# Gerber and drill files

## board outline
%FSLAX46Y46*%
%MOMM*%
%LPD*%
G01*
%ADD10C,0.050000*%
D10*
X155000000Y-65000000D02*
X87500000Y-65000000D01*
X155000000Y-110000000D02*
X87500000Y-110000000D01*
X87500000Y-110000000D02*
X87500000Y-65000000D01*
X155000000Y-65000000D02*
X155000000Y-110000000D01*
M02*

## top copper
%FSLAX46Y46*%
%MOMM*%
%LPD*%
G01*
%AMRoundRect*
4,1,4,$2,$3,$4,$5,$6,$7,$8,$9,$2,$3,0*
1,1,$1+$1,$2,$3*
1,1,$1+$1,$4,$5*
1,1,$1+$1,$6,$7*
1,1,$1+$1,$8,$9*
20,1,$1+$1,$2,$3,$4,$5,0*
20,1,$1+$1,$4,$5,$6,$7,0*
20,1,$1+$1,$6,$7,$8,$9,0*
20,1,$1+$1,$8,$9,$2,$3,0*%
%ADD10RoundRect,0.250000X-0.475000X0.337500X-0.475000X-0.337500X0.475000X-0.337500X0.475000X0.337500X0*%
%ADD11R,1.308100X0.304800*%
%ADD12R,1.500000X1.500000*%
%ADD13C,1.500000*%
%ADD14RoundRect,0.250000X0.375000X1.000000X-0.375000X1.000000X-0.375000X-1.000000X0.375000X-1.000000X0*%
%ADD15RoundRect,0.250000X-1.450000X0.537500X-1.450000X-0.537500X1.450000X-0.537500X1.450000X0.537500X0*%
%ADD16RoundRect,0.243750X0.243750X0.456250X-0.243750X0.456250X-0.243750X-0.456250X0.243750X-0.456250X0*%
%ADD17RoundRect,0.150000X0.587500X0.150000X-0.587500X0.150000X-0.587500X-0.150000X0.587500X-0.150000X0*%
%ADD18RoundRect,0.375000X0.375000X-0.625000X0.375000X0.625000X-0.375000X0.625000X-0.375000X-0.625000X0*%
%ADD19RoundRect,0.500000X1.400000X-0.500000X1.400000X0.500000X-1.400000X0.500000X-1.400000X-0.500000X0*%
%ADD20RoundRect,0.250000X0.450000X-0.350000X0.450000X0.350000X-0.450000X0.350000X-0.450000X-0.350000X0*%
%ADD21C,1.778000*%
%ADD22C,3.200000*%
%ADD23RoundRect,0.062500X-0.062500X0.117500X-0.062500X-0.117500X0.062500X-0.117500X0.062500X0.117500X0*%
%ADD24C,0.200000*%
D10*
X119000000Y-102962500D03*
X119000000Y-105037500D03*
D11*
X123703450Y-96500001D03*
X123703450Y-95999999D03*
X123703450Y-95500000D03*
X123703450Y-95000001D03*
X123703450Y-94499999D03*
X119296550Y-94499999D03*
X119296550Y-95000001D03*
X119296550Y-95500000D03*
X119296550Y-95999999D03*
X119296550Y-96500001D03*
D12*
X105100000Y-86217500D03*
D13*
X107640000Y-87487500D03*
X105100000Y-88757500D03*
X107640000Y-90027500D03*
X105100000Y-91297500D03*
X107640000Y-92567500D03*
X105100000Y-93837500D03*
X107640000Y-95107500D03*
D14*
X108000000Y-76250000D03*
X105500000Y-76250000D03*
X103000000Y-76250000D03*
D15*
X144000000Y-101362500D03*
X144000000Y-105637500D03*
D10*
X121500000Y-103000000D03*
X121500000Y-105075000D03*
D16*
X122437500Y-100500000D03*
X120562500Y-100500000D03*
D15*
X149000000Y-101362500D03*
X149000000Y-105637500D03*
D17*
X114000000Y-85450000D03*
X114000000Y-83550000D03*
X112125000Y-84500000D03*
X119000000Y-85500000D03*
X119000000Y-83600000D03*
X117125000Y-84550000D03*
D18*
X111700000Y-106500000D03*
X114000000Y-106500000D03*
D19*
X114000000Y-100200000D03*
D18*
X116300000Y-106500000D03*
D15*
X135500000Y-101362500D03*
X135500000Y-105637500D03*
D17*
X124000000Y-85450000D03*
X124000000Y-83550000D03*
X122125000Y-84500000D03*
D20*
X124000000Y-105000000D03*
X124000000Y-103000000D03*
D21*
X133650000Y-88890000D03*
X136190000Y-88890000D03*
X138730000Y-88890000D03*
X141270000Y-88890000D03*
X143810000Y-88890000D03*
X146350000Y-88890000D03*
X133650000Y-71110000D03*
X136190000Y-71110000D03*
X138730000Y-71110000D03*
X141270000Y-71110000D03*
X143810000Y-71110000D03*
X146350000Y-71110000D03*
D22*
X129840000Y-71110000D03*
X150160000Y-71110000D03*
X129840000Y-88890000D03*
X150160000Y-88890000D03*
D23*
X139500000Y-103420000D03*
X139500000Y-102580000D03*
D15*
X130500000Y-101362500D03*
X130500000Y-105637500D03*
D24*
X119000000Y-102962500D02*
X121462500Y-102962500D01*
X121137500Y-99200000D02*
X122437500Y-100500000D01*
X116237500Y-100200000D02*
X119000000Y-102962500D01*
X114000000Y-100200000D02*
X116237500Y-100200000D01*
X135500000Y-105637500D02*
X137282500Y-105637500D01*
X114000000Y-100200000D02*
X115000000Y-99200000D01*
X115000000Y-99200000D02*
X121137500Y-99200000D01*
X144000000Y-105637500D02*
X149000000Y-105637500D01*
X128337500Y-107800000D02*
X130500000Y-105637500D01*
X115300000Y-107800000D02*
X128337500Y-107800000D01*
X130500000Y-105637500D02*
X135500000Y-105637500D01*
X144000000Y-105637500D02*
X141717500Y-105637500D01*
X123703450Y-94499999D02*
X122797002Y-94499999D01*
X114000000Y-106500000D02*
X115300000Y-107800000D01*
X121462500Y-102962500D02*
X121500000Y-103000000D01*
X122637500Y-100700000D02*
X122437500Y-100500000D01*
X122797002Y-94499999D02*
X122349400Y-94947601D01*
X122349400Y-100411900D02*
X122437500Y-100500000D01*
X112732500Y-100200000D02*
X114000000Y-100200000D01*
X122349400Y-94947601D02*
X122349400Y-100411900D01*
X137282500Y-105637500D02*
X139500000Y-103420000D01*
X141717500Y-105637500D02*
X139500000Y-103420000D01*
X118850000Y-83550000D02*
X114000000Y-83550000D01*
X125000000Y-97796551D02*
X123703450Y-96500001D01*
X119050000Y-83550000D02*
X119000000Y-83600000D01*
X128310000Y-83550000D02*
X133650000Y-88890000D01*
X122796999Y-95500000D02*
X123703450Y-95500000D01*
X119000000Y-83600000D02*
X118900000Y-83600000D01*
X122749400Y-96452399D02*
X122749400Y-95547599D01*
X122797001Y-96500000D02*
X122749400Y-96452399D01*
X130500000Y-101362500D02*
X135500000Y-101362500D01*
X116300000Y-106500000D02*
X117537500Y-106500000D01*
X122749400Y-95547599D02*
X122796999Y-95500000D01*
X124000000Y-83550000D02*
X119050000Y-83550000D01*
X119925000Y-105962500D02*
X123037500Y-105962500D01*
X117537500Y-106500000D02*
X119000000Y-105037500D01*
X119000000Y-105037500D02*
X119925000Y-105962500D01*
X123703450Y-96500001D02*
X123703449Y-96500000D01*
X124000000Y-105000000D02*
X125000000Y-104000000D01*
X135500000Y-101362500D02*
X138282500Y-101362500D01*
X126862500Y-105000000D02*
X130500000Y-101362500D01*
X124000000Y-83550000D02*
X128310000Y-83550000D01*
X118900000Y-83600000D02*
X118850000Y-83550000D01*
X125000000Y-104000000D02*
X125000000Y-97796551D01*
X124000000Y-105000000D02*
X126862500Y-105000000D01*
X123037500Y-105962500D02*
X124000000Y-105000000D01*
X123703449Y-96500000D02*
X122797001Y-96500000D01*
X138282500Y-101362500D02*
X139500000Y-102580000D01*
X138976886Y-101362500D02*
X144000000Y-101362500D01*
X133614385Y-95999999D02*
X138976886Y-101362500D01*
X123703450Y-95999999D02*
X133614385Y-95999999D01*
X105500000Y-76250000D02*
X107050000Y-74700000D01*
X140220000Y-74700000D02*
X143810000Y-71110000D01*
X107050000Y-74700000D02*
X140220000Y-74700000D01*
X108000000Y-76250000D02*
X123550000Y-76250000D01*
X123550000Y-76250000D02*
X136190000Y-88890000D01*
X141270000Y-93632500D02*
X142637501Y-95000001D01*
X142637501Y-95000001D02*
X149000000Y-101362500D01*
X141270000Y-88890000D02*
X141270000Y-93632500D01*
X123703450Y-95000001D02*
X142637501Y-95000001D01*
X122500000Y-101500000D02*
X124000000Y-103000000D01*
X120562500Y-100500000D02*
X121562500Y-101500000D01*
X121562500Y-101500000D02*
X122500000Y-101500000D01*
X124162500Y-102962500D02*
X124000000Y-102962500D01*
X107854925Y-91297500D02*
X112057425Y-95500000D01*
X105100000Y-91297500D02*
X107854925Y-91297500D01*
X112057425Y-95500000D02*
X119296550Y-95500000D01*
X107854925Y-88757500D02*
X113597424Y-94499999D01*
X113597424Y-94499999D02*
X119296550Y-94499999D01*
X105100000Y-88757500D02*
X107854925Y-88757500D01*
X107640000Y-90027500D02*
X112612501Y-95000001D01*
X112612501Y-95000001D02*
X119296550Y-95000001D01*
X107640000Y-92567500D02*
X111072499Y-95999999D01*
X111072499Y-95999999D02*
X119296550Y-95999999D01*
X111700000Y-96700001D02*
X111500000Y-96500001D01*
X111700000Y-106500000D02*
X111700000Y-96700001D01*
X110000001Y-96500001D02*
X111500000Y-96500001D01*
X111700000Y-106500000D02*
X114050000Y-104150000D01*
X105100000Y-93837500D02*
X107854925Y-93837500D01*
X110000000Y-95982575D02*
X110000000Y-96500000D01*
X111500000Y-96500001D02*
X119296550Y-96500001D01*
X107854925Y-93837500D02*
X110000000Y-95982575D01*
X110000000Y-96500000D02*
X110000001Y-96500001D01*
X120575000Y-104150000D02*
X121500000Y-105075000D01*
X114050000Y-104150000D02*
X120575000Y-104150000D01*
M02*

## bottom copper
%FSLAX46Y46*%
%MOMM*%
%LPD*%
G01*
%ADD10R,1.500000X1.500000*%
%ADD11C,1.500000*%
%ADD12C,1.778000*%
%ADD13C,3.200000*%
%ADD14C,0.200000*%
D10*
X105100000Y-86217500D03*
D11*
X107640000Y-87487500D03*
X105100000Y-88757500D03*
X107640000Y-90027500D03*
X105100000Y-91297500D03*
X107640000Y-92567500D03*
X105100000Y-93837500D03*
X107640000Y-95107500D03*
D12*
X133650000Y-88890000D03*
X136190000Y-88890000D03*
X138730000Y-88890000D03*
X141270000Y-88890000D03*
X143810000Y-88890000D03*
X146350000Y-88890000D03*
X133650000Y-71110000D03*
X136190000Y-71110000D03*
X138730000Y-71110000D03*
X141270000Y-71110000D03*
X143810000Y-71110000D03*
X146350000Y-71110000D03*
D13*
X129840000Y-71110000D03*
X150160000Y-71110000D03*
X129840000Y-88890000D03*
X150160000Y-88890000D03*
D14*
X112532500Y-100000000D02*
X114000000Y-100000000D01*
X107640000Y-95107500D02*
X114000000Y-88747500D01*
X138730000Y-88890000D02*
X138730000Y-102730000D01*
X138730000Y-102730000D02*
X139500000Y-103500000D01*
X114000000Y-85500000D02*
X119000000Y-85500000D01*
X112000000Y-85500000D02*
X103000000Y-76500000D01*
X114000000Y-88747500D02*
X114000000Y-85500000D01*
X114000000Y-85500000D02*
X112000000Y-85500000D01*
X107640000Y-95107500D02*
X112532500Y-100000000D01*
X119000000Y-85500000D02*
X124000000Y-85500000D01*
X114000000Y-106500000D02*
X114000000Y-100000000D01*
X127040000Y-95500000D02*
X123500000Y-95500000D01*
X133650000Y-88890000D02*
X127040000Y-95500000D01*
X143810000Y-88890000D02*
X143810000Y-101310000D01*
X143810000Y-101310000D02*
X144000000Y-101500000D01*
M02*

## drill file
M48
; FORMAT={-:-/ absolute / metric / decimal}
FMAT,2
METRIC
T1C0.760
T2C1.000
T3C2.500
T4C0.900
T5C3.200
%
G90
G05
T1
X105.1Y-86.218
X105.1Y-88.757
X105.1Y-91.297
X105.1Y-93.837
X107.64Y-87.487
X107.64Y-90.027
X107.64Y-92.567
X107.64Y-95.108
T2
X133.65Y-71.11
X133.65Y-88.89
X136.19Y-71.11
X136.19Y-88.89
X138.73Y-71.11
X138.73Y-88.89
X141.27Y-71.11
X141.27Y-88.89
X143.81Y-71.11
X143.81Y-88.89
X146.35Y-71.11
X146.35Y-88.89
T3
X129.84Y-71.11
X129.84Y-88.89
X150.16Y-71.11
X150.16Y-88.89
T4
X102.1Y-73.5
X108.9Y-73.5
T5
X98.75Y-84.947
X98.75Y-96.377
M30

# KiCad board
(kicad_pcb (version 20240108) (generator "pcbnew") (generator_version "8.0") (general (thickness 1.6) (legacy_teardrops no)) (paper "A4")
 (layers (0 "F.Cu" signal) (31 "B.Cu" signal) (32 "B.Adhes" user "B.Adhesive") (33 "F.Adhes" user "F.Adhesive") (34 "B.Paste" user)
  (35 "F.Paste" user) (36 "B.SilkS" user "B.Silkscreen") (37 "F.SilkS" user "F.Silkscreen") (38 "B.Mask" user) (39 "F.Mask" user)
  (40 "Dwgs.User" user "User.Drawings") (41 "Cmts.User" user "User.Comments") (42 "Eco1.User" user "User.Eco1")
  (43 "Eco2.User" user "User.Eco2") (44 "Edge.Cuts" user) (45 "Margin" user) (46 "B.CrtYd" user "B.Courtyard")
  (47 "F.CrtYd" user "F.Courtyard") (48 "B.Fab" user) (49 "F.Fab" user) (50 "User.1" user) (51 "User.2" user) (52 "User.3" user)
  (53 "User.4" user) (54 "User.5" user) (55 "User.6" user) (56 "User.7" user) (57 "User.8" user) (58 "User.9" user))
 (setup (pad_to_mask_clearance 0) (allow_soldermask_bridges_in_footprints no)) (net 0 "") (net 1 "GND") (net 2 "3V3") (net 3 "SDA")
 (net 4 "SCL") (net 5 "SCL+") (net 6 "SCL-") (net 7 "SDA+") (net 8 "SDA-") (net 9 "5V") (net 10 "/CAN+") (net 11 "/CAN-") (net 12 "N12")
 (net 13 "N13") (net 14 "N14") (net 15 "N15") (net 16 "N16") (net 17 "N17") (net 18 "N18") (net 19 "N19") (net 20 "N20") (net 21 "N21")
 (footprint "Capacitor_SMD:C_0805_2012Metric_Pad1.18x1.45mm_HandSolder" (layer "F.Cu") (at 119 104 -90)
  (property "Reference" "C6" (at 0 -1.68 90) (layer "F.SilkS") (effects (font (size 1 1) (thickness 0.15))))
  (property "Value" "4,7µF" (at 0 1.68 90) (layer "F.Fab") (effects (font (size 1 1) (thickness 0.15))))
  (pad "1" smd roundrect (at -1.0375 0 270) (size 1.175 1.45) (layers "F.Cu" "F.Paste" "F.Mask") (roundrect_rratio 0.212766) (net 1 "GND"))
  (pad "2" smd roundrect (at 1.0375 0 270) (size 1.175 1.45) (layers "F.Cu" "F.Paste" "F.Mask") (roundrect_rratio 0.212766) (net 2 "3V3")))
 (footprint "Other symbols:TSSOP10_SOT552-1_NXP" (layer "F.Cu") (at 121.5 95.5 180)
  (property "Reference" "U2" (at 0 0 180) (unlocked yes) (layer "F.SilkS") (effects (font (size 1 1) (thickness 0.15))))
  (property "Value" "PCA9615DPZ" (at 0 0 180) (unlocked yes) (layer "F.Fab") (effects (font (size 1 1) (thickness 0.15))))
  (pad "1" smd rect (at -2.20345 -1.000001 180) (size 1.3081 0.3048) (layers "F.Cu" "F.Paste" "F.Mask") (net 2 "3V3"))
  (pad "2" smd rect (at -2.20345 -0.499999 180) (size 1.3081 0.3048) (layers "F.Cu" "F.Paste" "F.Mask") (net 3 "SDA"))
  (pad "3" smd rect (at -2.20345 0 180) (size 1.3081 0.3048) (layers "F.Cu" "F.Paste" "F.Mask") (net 2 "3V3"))
  (pad "4" smd rect (at -2.20345 0.499999 180) (size 1.3081 0.3048) (layers "F.Cu" "F.Paste" "F.Mask") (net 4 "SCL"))
  (pad "5" smd rect (at -2.20345 1.000001 180) (size 1.3081 0.3048) (layers "F.Cu" "F.Paste" "F.Mask") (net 1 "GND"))
  (pad "6" smd rect (at 2.20345 1.000001 180) (size 1.3081 0.3048) (layers "F.Cu" "F.Paste" "F.Mask") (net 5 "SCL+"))
  (pad "7" smd rect (at 2.20345 0.499999 180) (size 1.3081 0.3048) (layers "F.Cu" "F.Paste" "F.Mask") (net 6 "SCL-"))
  (pad "8" smd rect (at 2.20345 0 180) (size 1.3081 0.3048) (layers "F.Cu" "F.Paste" "F.Mask") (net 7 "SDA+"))
  (pad "9" smd rect (at 2.20345 -0.499999 180) (size 1.3081 0.3048) (layers "F.Cu" "F.Paste" "F.Mask") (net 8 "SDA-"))
  (pad "10" smd rect (at 2.20345 -1.000001 180) (size 1.3081 0.3048) (layers "F.Cu" "F.Paste" "F.Mask") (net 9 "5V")))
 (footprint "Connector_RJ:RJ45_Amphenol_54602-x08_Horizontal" (layer "F.Cu") (at 105.1 86.2175 -90)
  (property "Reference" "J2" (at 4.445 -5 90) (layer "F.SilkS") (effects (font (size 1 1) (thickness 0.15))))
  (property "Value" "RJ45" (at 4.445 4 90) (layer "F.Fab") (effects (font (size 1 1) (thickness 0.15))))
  (pad "" np_thru_hole circle (at -1.27 6.35 270) (size 3.2 3.2) (drill 3.2) (layers "*.Cu" "*.Mask"))
  (pad "" np_thru_hole circle (at 10.16 6.35 270) (size 3.2 3.2) (drill 3.2) (layers "*.Cu" "*.Mask"))
  (pad "1" thru_hole rect (at 0 0 270) (size 1.5 1.5) (drill 0.76) (layers "*.Cu" "*.Mask") (remove_unused_layers no) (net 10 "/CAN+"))
  (pad "2" thru_hole circle (at 1.27 -2.54 270) (size 1.5 1.5) (drill 0.76) (layers "*.Cu" "*.Mask") (remove_unused_layers no)
   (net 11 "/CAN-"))
  (pad "3" thru_hole circle (at 2.54 0 270) (size 1.5 1.5) (drill 0.76) (layers "*.Cu" "*.Mask") (remove_unused_layers no) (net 5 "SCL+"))
  (pad "4" thru_hole circle (at 3.81 -2.54 270) (size 1.5 1.5) (drill 0.76) (layers "*.Cu" "*.Mask") (remove_unused_layers no)
   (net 6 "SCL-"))
  (pad "5" thru_hole circle (at 5.08 0 270) (size 1.5 1.5) (drill 0.76) (layers "*.Cu" "*.Mask") (remove_unused_layers no) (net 7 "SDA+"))
  (pad "6" thru_hole circle (at 6.35 -2.54 270) (size 1.5 1.5) (drill 0.76) (layers "*.Cu" "*.Mask") (remove_unused_layers no)
   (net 8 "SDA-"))
  (pad "7" thru_hole circle (at 7.62 0 270) (size 1.5 1.5) (drill 0.76) (layers "*.Cu" "*.Mask") (remove_unused_layers no) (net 9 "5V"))
  (pad "8" thru_hole circle (at 8.89 -2.54 270) (size 1.5 1.5) (drill 0.76) (layers "*.Cu" "*.Mask") (remove_unused_layers no) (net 1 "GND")))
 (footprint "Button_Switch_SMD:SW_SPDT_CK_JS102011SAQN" (layer "F.Cu") (at 105.5 73.5 180)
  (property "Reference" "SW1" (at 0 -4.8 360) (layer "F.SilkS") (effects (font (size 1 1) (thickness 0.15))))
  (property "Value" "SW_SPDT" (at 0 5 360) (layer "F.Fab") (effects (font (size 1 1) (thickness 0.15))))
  (pad "" np_thru_hole circle (at -3.4 0 180) (size 0.9 0.9) (drill 0.9) (layers "*.Cu" "*.Mask"))
  (pad "" np_thru_hole circle (at 3.4 0 180) (size 0.9 0.9) (drill 0.9) (layers "*.Cu" "*.Mask"))
  (pad "1" smd roundrect (at -2.5 -2.75 180) (size 1.25 2.5) (layers "F.Cu" "F.Paste" "F.Mask") (roundrect_rratio 0.2) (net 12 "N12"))
  (pad "2" smd roundrect (at 0 -2.75 180) (size 1.25 2.5) (layers "F.Cu" "F.Paste" "F.Mask") (roundrect_rratio 0.2) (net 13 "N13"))
  (pad "3" smd roundrect (at 2.5 -2.75 180) (size 1.25 2.5) (layers "F.Cu" "F.Paste" "F.Mask") (roundrect_rratio 0.2) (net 1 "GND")))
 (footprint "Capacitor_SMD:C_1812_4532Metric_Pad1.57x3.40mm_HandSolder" (layer "F.Cu") (at 144 103.5 -90)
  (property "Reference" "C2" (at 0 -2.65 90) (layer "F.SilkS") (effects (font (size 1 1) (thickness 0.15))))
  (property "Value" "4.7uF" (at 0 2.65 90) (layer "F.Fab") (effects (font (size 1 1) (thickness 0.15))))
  (pad "1" smd roundrect (at -2.1375 0 270) (size 1.575 3.4) (layers "F.Cu" "F.Paste" "F.Mask") (roundrect_rratio 0.15873) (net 3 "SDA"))
  (pad "2" smd roundrect (at 2.1375 0 270) (size 1.575 3.4) (layers "F.Cu" "F.Paste" "F.Mask") (roundrect_rratio 0.15873) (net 1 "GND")))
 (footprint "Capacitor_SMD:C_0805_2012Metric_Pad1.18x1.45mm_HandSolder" (layer "F.Cu") (at 121.5 104.0375 -90)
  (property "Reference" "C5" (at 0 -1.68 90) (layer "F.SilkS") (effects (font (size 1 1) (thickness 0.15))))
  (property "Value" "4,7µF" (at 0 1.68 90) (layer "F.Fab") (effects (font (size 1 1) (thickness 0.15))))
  (pad "1" smd roundrect (at -1.0375 0 270) (size 1.175 1.45) (layers "F.Cu" "F.Paste" "F.Mask") (roundrect_rratio 0.212766) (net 1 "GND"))
  (pad "2" smd roundrect (at 1.0375 0 270) (size 1.175 1.45) (layers "F.Cu" "F.Paste" "F.Mask") (roundrect_rratio 0.212766) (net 9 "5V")))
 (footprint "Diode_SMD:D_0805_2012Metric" (layer "F.Cu") (at 121.5 100.5 180)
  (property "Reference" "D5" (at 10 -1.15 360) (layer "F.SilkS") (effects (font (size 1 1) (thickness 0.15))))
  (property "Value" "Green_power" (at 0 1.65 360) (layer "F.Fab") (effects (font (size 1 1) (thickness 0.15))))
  (pad "1" smd roundrect (at -0.9375 0 180) (size 0.975 1.4) (layers "F.Cu" "F.Paste" "F.Mask") (roundrect_rratio 0.25) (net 1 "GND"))
  (pad "2" smd roundrect (at 0.9375 0 180) (size 0.975 1.4) (layers "F.Cu" "F.Paste" "F.Mask") (roundrect_rratio 0.25) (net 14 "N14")))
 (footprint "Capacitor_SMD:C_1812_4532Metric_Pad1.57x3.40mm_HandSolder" (layer "F.Cu") (at 149 103.5 -90)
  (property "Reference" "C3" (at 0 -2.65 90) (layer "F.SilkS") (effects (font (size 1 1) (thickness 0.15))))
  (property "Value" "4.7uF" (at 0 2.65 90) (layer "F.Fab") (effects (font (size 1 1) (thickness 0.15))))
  (pad "1" smd roundrect (at -2.1375 0 270) (size 1.575 3.4) (layers "F.Cu" "F.Paste" "F.Mask") (roundrect_rratio 0.15873) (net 4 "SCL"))
  (pad "2" smd roundrect (at 2.1375 0 270) (size 1.575 3.4) (layers "F.Cu" "F.Paste" "F.Mask") (roundrect_rratio 0.15873) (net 1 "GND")))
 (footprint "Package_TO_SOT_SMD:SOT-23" (layer "F.Cu") (at 113.0625 84.5 180)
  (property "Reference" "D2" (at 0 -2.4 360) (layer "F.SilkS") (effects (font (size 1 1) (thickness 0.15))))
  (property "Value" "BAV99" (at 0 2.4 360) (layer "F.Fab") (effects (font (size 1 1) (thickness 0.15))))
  (pad "1" smd roundrect (at -0.9375 -0.95 180) (size 1.475 0.6) (layers "F.Cu" "F.Paste" "F.Mask") (roundrect_rratio 0.25) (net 1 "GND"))
  (pad "2" smd roundrect (at -0.9375 0.95 180) (size 1.475 0.6) (layers "F.Cu" "F.Paste" "F.Mask") (roundrect_rratio 0.25) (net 2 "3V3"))
  (pad "3" smd roundrect (at 0.9375 0 180) (size 1.475 0.6) (layers "F.Cu" "F.Paste" "F.Mask") (roundrect_rratio 0.25) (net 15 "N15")))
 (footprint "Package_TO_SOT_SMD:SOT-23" (layer "F.Cu") (at 118.0625 84.55 180)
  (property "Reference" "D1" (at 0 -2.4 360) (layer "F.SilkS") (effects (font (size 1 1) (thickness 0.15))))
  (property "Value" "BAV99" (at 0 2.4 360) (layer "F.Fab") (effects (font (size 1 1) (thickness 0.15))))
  (pad "1" smd roundrect (at -0.9375 -0.95 180) (size 1.475 0.6) (layers "F.Cu" "F.Paste" "F.Mask") (roundrect_rratio 0.25) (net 1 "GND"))
  (pad "2" smd roundrect (at -0.9375 0.95 180) (size 1.475 0.6) (layers "F.Cu" "F.Paste" "F.Mask") (roundrect_rratio 0.25) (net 2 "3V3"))
  (pad "3" smd roundrect (at 0.9375 0 180) (size 1.475 0.6) (layers "F.Cu" "F.Paste" "F.Mask") (roundrect_rratio 0.25) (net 4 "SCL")))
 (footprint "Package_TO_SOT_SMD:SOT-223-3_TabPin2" (layer "F.Cu") (at 114 103.35 90)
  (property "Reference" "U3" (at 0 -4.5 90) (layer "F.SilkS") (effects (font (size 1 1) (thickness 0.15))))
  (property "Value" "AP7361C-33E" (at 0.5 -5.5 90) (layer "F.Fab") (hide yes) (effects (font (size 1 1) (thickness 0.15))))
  (pad "1" smd roundrect (at -3.15 -2.3 90) (size 2 1.5) (layers "F.Cu" "F.Paste" "F.Mask") (roundrect_rratio 0.25) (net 9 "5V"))
  (pad "2" smd roundrect (at -3.15 0 90) (size 2 1.5) (layers "F.Cu" "F.Paste" "F.Mask") (roundrect_rratio 0.25) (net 1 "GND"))
  (pad "2" smd roundrect (at 3.15 0 90) (size 2 3.8) (layers "F.Cu" "F.Paste" "F.Mask") (roundrect_rratio 0.25) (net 1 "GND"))
  (pad "3" smd roundrect (at -3.15 2.3 90) (size 2 1.5) (layers "F.Cu" "F.Paste" "F.Mask") (roundrect_rratio 0.25) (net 2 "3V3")))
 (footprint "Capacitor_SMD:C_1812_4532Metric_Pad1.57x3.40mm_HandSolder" (layer "F.Cu") (at 135.5 103.5 -90)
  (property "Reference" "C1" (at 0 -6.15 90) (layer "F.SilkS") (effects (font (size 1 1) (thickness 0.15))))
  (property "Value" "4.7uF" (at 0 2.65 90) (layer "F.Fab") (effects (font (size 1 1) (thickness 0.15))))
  (pad "1" smd roundrect (at -2.1375 0 270) (size 1.575 3.4) (layers "F.Cu" "F.Paste" "F.Mask") (roundrect_rratio 0.15873) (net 2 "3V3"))
  (pad "2" smd roundrect (at 2.1375 0 270) (size 1.575 3.4) (layers "F.Cu" "F.Paste" "F.Mask") (roundrect_rratio 0.15873) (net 1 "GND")))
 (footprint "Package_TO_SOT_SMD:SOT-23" (layer "F.Cu") (at 123.0625 84.5 180)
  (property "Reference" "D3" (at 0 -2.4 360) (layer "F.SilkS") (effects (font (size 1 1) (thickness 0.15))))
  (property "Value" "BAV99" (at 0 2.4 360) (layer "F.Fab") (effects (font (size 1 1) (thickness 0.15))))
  (pad "1" smd roundrect (at -0.9375 -0.95 180) (size 1.475 0.6) (layers "F.Cu" "F.Paste" "F.Mask") (roundrect_rratio 0.25) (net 1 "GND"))
  (pad "2" smd roundrect (at -0.9375 0.95 180) (size 1.475 0.6) (layers "F.Cu" "F.Paste" "F.Mask") (roundrect_rratio 0.25) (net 2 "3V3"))
  (pad "3" smd roundrect (at 0.9375 0 180) (size 1.475 0.6) (layers "F.Cu" "F.Paste" "F.Mask") (roundrect_rratio 0.25) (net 3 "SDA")))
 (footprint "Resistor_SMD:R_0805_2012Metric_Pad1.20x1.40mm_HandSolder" (layer "F.Cu") (at 124 104 90)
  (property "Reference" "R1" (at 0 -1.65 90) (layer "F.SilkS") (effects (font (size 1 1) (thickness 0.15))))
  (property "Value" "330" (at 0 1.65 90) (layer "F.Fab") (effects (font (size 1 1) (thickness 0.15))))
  (pad "1" smd roundrect (at -1 0 90) (size 1.2 1.4) (layers "F.Cu" "F.Paste" "F.Mask") (roundrect_rratio 0.208333) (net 2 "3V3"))
  (pad "2" smd roundrect (at 1 0 90) (size 1.2 1.4) (layers "F.Cu" "F.Paste" "F.Mask") (roundrect_rratio 0.208333) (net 14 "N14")))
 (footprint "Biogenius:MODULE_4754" (layer "F.Cu") (at 140 80)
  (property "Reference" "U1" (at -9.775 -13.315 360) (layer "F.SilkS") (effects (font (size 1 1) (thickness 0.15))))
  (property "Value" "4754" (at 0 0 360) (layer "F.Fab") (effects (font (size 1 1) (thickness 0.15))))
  (pad "JP1_1" thru_hole circle (at -6.35 8.89) (size 1.778 1.778) (drill 1) (layers "*.Cu" "*.Mask") (remove_unused_layers no)
   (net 2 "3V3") (solder_mask_margin 0.102))
  (pad "JP1_2" thru_hole circle (at -3.81 8.89) (size 1.778 1.778) (drill 1) (layers "*.Cu" "*.Mask") (remove_unused_layers no)
   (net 12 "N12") (solder_mask_margin 0.102))
  (pad "JP1_3" thru_hole circle (at -1.27 8.89) (size 1.778 1.778) (drill 1) (layers "*.Cu" "*.Mask") (remove_unused_layers no)
   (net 1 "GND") (solder_mask_margin 0.102))
  (pad "JP1_4" thru_hole circle (at 1.27 8.89) (size 1.778 1.778) (drill 1) (layers "*.Cu" "*.Mask") (remove_unused_layers no) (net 4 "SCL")
   (solder_mask_margin 0.102))
  (pad "JP1_5" thru_hole circle (at 3.81 8.89) (size 1.778 1.778) (drill 1) (layers "*.Cu" "*.Mask") (remove_unused_layers no) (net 3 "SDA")
   (solder_mask_margin 0.102))
  (pad "JP1_6" thru_hole circle (at 6.35 8.89) (size 1.778 1.778) (drill 1) (layers "*.Cu" "*.Mask") (remove_unused_layers no)
   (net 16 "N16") (solder_mask_margin 0.102))
  (pad "JP2_1" thru_hole circle (at -6.35 -8.89) (size 1.778 1.778) (drill 1) (layers "*.Cu" "*.Mask") (remove_unused_layers no)
   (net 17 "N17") (solder_mask_margin 0.102))
  (pad "JP2_2" thru_hole circle (at -3.81 -8.89) (size 1.778 1.778) (drill 1) (layers "*.Cu" "*.Mask") (remove_unused_layers no)
   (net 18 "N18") (solder_mask_margin 0.102))
  (pad "JP2_3" thru_hole circle (at -1.27 -8.89) (size 1.778 1.778) (drill 1) (layers "*.Cu" "*.Mask") (remove_unused_layers no)
   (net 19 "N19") (solder_mask_margin 0.102))
  (pad "JP2_4" thru_hole circle (at 1.27 -8.89) (size 1.778 1.778) (drill 1) (layers "*.Cu" "*.Mask") (remove_unused_layers no)
   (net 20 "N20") (solder_mask_margin 0.102))
  (pad "JP2_5" thru_hole circle (at 3.81 -8.89) (size 1.778 1.778) (drill 1) (layers "*.Cu" "*.Mask") (remove_unused_layers no)
   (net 13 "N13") (solder_mask_margin 0.102))
  (pad "JP2_6" thru_hole circle (at 6.35 -8.89) (size 1.778 1.778) (drill 1) (layers "*.Cu" "*.Mask") (remove_unused_layers no)
   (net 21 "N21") (solder_mask_margin 0.102))
  (pad "P1" thru_hole circle (at -10.16 -8.89) (size 3.2 3.2) (drill 2.5) (layers "*.Cu" "*.Mask") (remove_unused_layers no)
   (solder_mask_margin 0.102))
  (pad "P2" thru_hole circle (at 10.16 -8.89) (size 3.2 3.2) (drill 2.5) (layers "*.Cu" "*.Mask") (remove_unused_layers no)
   (solder_mask_margin 0.102))
  (pad "P3" thru_hole circle (at -10.16 8.89) (size 3.2 3.2) (drill 2.5) (layers "*.Cu" "*.Mask") (remove_unused_layers no)
   (solder_mask_margin 0.102))
  (pad "P4" thru_hole circle (at 10.16 8.89) (size 3.2 3.2) (drill 2.5) (layers "*.Cu" "*.Mask") (remove_unused_layers no)
   (solder_mask_margin 0.102)))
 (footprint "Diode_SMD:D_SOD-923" (layer "F.Cu") (at 139.5 103 90)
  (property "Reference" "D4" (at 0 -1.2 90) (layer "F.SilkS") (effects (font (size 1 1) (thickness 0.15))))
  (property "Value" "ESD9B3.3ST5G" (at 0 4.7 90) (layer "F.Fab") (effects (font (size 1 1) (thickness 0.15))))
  (pad "1" smd roundrect (at -0.42 0 270) (size 0.36 0.25) (layers "F.Cu" "F.Paste" "F.Mask") (roundrect_rratio 0.25) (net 1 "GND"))
  (pad "2" smd roundrect (at 0.42 0 270) (size 0.36 0.25) (layers "F.Cu" "F.Paste" "F.Mask") (roundrect_rratio 0.25) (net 2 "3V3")))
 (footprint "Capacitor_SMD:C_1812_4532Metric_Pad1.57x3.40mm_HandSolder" (layer "F.Cu") (at 130.5 103.5 -90)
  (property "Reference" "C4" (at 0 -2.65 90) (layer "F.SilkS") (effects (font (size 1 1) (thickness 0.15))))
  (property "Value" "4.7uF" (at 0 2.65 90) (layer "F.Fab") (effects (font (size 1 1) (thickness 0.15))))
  (pad "1" smd roundrect (at -2.1375 0 270) (size 1.575 3.4) (layers "F.Cu" "F.Paste" "F.Mask") (roundrect_rratio 0.15873) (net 2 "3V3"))
  (pad "2" smd roundrect (at 2.1375 0 270) (size 1.575 3.4) (layers "F.Cu" "F.Paste" "F.Mask") (roundrect_rratio 0.15873) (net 1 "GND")))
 (gr_line (start 155 65) (end 87.5 65) (stroke (width 0.05) (type default)) (layer "Edge.Cuts"))
 (gr_line (start 155 110) (end 87.5 110) (stroke (width 0.05) (type default)) (layer "Edge.Cuts"))
 (gr_line (start 87.5 110) (end 87.5 65) (stroke (width 0.05) (type default)) (layer "Edge.Cuts"))
 (gr_line (start 155 65) (end 155 110) (stroke (width 0.05) (type default)) (layer "Edge.Cuts"))
 (segment (start 119 102.9625) (end 121.4625 102.9625) (width 0.2) (layer "F.Cu") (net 1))
 (segment (start 121.1375 99.2) (end 122.4375 100.5) (width 0.2) (layer "F.Cu") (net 1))
 (segment (start 116.2375 100.2) (end 119 102.9625) (width 0.2) (layer "F.Cu") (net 1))
 (segment (start 114 100.2) (end 116.2375 100.2) (width 0.2) (layer "F.Cu") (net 1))
 (segment (start 135.5 105.6375) (end 137.2825 105.6375) (width 0.2) (layer "F.Cu") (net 1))
 (segment (start 114 100.2) (end 115 99.2) (width 0.2) (layer "F.Cu") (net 1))
 (segment (start 115 99.2) (end 121.1375 99.2) (width 0.2) (layer "F.Cu") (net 1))
 (segment (start 144 105.6375) (end 149 105.6375) (width 0.2) (layer "F.Cu") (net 1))
 (segment (start 128.3375 107.8) (end 130.5 105.6375) (width 0.2) (layer "F.Cu") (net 1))
 (segment (start 115.3 107.8) (end 128.3375 107.8) (width 0.2) (layer "F.Cu") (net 1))
 (segment (start 130.5 105.6375) (end 135.5 105.6375) (width 0.2) (layer "F.Cu") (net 1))
 (segment (start 144 105.6375) (end 141.7175 105.6375) (width 0.2) (layer "F.Cu") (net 1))
 (segment (start 123.70345 94.499999) (end 122.797002 94.499999) (width 0.2) (layer "F.Cu") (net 1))
 (segment (start 114 106.5) (end 115.3 107.8) (width 0.2) (layer "F.Cu") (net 1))
 (segment (start 121.4625 102.9625) (end 121.5 103) (width 0.2) (layer "F.Cu") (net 1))
 (segment (start 122.6375 100.7) (end 122.4375 100.5) (width 0.2) (layer "F.Cu") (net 1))
 (segment (start 122.797002 94.499999) (end 122.3494 94.947601) (width 0.2) (layer "F.Cu") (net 1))
 (segment (start 122.3494 100.4119) (end 122.4375 100.5) (width 0.2) (layer "F.Cu") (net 1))
 (segment (start 112.7325 100.2) (end 114 100.2) (width 0.2) (layer "F.Cu") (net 1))
 (segment (start 122.3494 94.947601) (end 122.3494 100.4119) (width 0.2) (layer "F.Cu") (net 1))
 (segment (start 137.2825 105.6375) (end 139.5 103.42) (width 0.2) (layer "F.Cu") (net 1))
 (segment (start 141.7175 105.6375) (end 139.5 103.42) (width 0.2) (layer "F.Cu") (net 1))
 (segment (start 112.5325 100) (end 114 100) (width 0.2) (layer "B.Cu") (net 1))
 (segment (start 107.64 95.1075) (end 114 88.7475) (width 0.2) (layer "B.Cu") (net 1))
 (segment (start 138.73 88.89) (end 138.73 102.73) (width 0.2) (layer "B.Cu") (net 1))
 (segment (start 138.73 102.73) (end 139.5 103.5) (width 0.2) (layer "B.Cu") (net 1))
 (segment (start 114 85.5) (end 119 85.5) (width 0.2) (layer "B.Cu") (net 1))
 (segment (start 112 85.5) (end 103 76.5) (width 0.2) (layer "B.Cu") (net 1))
 (segment (start 114 88.7475) (end 114 85.5) (width 0.2) (layer "B.Cu") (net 1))
 (segment (start 114 85.5) (end 112 85.5) (width 0.2) (layer "B.Cu") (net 1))
 (segment (start 107.64 95.1075) (end 112.5325 100) (width 0.2) (layer "B.Cu") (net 1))
 (segment (start 119 85.5) (end 124 85.5) (width 0.2) (layer "B.Cu") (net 1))
 (segment (start 114 106.5) (end 114 100) (width 0.2) (layer "B.Cu") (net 1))
 (segment (start 118.85 83.55) (end 114 83.55) (width 0.2) (layer "F.Cu") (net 2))
 (segment (start 125 97.796551) (end 123.70345 96.500001) (width 0.2) (layer "F.Cu") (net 2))
 (segment (start 119.05 83.55) (end 119 83.6) (width 0.2) (layer "F.Cu") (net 2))
 (segment (start 128.31 83.55) (end 133.65 88.89) (width 0.2) (layer "F.Cu") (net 2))
 (segment (start 122.796999 95.5) (end 123.70345 95.5) (width 0.2) (layer "F.Cu") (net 2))
 (segment (start 119 83.6) (end 118.9 83.6) (width 0.2) (layer "F.Cu") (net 2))
 (segment (start 122.7494 96.452399) (end 122.7494 95.547599) (width 0.2) (layer "F.Cu") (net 2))
 (segment (start 122.797001 96.5) (end 122.7494 96.452399) (width 0.2) (layer "F.Cu") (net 2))
 (segment (start 130.5 101.3625) (end 135.5 101.3625) (width 0.2) (layer "F.Cu") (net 2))
 (segment (start 116.3 106.5) (end 117.5375 106.5) (width 0.2) (layer "F.Cu") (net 2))
 (segment (start 122.7494 95.547599) (end 122.796999 95.5) (width 0.2) (layer "F.Cu") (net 2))
 (segment (start 124 83.55) (end 119.05 83.55) (width 0.2) (layer "F.Cu") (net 2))
 (segment (start 119.925 105.9625) (end 123.0375 105.9625) (width 0.2) (layer "F.Cu") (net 2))
 (segment (start 117.5375 106.5) (end 119 105.0375) (width 0.2) (layer "F.Cu") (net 2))
 (segment (start 119 105.0375) (end 119.925 105.9625) (width 0.2) (layer "F.Cu") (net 2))
 (segment (start 123.70345 96.500001) (end 123.703449 96.5) (width 0.2) (layer "F.Cu") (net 2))
 (segment (start 124 105) (end 125 104) (width 0.2) (layer "F.Cu") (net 2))
 (segment (start 135.5 101.3625) (end 138.2825 101.3625) (width 0.2) (layer "F.Cu") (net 2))
 (segment (start 126.8625 105) (end 130.5 101.3625) (width 0.2) (layer "F.Cu") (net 2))
 (segment (start 124 83.55) (end 128.31 83.55) (width 0.2) (layer "F.Cu") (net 2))
 (segment (start 118.9 83.6) (end 118.85 83.55) (width 0.2) (layer "F.Cu") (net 2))
 (segment (start 125 104) (end 125 97.796551) (width 0.2) (layer "F.Cu") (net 2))
 (segment (start 124 105) (end 126.8625 105) (width 0.2) (layer "F.Cu") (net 2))
 (segment (start 123.0375 105.9625) (end 124 105) (width 0.2) (layer "F.Cu") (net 2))
 (segment (start 123.703449 96.5) (end 122.797001 96.5) (width 0.2) (layer "F.Cu") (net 2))
 (segment (start 138.2825 101.3625) (end 139.5 102.58) (width 0.2) (layer "F.Cu") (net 2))
 (segment (start 127.04 95.5) (end 123.5 95.5) (width 0.2) (layer "B.Cu") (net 2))
 (segment (start 133.65 88.89) (end 127.04 95.5) (width 0.2) (layer "B.Cu") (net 2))
 (segment (start 138.976886 101.3625) (end 144 101.3625) (width 0.2) (layer "F.Cu") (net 3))
 (segment (start 133.614385 95.999999) (end 138.976886 101.3625) (width 0.2) (layer "F.Cu") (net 3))
 (segment (start 123.70345 95.999999) (end 133.614385 95.999999) (width 0.2) (layer "F.Cu") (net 3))
 (segment (start 143.81 88.89) (end 143.81 101.31) (width 0.2) (layer "B.Cu") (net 3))
 (segment (start 143.81 101.31) (end 144 101.5) (width 0.2) (layer "B.Cu") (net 3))
 (segment (start 105.5 76.25) (end 107.05 74.7) (width 0.2) (layer "F.Cu") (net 13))
 (segment (start 140.22 74.7) (end 143.81 71.11) (width 0.2) (layer "F.Cu") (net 13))
 (segment (start 107.05 74.7) (end 140.22 74.7) (width 0.2) (layer "F.Cu") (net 13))
 (segment (start 108 76.25) (end 123.55 76.25) (width 0.2) (layer "F.Cu") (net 12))
 (segment (start 123.55 76.25) (end 136.19 88.89) (width 0.2) (layer "F.Cu") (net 12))
 (segment (start 141.27 93.6325) (end 142.637501 95.000001) (width 0.2) (layer "F.Cu") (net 4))
 (segment (start 142.637501 95.000001) (end 149 101.3625) (width 0.2) (layer "F.Cu") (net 4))
 (segment (start 141.27 88.89) (end 141.27 93.6325) (width 0.2) (layer "F.Cu") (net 4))
 (segment (start 123.70345 95.000001) (end 142.637501 95.000001) (width 0.2) (layer "F.Cu") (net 4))
 (segment (start 122.5 101.5) (end 124 103) (width 0.2) (layer "F.Cu") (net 14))
 (segment (start 120.5625 100.5) (end 121.5625 101.5) (width 0.2) (layer "F.Cu") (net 14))
 (segment (start 121.5625 101.5) (end 122.5 101.5) (width 0.2) (layer "F.Cu") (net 14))
 (segment (start 124.1625 102.9625) (end 124 102.9625) (width 0.2) (layer "F.Cu") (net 14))
 (segment (start 107.854925 91.2975) (end 112.057425 95.5) (width 0.2) (layer "F.Cu") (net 7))
 (segment (start 105.1 91.2975) (end 107.854925 91.2975) (width 0.2) (layer "F.Cu") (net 7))
 (segment (start 112.057425 95.5) (end 119.29655 95.5) (width 0.2) (layer "F.Cu") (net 7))
 (segment (start 107.854925 88.7575) (end 113.597424 94.499999) (width 0.2) (layer "F.Cu") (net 5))
 (segment (start 113.597424 94.499999) (end 119.29655 94.499999) (width 0.2) (layer "F.Cu") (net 5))
 (segment (start 105.1 88.7575) (end 107.854925 88.7575) (width 0.2) (layer "F.Cu") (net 5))
 (segment (start 107.64 90.0275) (end 112.612501 95.000001) (width 0.2) (layer "F.Cu") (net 6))
 (segment (start 112.612501 95.000001) (end 119.29655 95.000001) (width 0.2) (layer "F.Cu") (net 6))
 (segment (start 107.64 92.5675) (end 111.072499 95.999999) (width 0.2) (layer "F.Cu") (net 8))
 (segment (start 111.072499 95.999999) (end 119.29655 95.999999) (width 0.2) (layer "F.Cu") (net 8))
 (segment (start 111.7 96.700001) (end 111.5 96.500001) (width 0.2) (layer "F.Cu") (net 9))
 (segment (start 111.7 106.5) (end 111.7 96.700001) (width 0.2) (layer "F.Cu") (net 9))
 (segment (start 110.000001 96.500001) (end 111.5 96.500001) (width 0.2) (layer "F.Cu") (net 9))
 (segment (start 111.7 106.5) (end 114.05 104.15) (width 0.2) (layer "F.Cu") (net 9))
 (segment (start 105.1 93.8375) (end 107.854925 93.8375) (width 0.2) (layer "F.Cu") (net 9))
 (segment (start 110 95.982575) (end 110 96.5) (width 0.2) (layer "F.Cu") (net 9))
 (segment (start 111.5 96.500001) (end 119.29655 96.500001) (width 0.2) (layer "F.Cu") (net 9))
 (segment (start 107.854925 93.8375) (end 110 95.982575) (width 0.2) (layer "F.Cu") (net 9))
 (segment (start 110 96.5) (end 110.000001 96.500001) (width 0.2) (layer "F.Cu") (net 9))
 (segment (start 120.575 104.15) (end 121.5 105.075) (width 0.2) (layer "F.Cu") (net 9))
 (segment (start 114.05 104.15) (end 120.575 104.15) (width 0.2) (layer "F.Cu") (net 9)))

